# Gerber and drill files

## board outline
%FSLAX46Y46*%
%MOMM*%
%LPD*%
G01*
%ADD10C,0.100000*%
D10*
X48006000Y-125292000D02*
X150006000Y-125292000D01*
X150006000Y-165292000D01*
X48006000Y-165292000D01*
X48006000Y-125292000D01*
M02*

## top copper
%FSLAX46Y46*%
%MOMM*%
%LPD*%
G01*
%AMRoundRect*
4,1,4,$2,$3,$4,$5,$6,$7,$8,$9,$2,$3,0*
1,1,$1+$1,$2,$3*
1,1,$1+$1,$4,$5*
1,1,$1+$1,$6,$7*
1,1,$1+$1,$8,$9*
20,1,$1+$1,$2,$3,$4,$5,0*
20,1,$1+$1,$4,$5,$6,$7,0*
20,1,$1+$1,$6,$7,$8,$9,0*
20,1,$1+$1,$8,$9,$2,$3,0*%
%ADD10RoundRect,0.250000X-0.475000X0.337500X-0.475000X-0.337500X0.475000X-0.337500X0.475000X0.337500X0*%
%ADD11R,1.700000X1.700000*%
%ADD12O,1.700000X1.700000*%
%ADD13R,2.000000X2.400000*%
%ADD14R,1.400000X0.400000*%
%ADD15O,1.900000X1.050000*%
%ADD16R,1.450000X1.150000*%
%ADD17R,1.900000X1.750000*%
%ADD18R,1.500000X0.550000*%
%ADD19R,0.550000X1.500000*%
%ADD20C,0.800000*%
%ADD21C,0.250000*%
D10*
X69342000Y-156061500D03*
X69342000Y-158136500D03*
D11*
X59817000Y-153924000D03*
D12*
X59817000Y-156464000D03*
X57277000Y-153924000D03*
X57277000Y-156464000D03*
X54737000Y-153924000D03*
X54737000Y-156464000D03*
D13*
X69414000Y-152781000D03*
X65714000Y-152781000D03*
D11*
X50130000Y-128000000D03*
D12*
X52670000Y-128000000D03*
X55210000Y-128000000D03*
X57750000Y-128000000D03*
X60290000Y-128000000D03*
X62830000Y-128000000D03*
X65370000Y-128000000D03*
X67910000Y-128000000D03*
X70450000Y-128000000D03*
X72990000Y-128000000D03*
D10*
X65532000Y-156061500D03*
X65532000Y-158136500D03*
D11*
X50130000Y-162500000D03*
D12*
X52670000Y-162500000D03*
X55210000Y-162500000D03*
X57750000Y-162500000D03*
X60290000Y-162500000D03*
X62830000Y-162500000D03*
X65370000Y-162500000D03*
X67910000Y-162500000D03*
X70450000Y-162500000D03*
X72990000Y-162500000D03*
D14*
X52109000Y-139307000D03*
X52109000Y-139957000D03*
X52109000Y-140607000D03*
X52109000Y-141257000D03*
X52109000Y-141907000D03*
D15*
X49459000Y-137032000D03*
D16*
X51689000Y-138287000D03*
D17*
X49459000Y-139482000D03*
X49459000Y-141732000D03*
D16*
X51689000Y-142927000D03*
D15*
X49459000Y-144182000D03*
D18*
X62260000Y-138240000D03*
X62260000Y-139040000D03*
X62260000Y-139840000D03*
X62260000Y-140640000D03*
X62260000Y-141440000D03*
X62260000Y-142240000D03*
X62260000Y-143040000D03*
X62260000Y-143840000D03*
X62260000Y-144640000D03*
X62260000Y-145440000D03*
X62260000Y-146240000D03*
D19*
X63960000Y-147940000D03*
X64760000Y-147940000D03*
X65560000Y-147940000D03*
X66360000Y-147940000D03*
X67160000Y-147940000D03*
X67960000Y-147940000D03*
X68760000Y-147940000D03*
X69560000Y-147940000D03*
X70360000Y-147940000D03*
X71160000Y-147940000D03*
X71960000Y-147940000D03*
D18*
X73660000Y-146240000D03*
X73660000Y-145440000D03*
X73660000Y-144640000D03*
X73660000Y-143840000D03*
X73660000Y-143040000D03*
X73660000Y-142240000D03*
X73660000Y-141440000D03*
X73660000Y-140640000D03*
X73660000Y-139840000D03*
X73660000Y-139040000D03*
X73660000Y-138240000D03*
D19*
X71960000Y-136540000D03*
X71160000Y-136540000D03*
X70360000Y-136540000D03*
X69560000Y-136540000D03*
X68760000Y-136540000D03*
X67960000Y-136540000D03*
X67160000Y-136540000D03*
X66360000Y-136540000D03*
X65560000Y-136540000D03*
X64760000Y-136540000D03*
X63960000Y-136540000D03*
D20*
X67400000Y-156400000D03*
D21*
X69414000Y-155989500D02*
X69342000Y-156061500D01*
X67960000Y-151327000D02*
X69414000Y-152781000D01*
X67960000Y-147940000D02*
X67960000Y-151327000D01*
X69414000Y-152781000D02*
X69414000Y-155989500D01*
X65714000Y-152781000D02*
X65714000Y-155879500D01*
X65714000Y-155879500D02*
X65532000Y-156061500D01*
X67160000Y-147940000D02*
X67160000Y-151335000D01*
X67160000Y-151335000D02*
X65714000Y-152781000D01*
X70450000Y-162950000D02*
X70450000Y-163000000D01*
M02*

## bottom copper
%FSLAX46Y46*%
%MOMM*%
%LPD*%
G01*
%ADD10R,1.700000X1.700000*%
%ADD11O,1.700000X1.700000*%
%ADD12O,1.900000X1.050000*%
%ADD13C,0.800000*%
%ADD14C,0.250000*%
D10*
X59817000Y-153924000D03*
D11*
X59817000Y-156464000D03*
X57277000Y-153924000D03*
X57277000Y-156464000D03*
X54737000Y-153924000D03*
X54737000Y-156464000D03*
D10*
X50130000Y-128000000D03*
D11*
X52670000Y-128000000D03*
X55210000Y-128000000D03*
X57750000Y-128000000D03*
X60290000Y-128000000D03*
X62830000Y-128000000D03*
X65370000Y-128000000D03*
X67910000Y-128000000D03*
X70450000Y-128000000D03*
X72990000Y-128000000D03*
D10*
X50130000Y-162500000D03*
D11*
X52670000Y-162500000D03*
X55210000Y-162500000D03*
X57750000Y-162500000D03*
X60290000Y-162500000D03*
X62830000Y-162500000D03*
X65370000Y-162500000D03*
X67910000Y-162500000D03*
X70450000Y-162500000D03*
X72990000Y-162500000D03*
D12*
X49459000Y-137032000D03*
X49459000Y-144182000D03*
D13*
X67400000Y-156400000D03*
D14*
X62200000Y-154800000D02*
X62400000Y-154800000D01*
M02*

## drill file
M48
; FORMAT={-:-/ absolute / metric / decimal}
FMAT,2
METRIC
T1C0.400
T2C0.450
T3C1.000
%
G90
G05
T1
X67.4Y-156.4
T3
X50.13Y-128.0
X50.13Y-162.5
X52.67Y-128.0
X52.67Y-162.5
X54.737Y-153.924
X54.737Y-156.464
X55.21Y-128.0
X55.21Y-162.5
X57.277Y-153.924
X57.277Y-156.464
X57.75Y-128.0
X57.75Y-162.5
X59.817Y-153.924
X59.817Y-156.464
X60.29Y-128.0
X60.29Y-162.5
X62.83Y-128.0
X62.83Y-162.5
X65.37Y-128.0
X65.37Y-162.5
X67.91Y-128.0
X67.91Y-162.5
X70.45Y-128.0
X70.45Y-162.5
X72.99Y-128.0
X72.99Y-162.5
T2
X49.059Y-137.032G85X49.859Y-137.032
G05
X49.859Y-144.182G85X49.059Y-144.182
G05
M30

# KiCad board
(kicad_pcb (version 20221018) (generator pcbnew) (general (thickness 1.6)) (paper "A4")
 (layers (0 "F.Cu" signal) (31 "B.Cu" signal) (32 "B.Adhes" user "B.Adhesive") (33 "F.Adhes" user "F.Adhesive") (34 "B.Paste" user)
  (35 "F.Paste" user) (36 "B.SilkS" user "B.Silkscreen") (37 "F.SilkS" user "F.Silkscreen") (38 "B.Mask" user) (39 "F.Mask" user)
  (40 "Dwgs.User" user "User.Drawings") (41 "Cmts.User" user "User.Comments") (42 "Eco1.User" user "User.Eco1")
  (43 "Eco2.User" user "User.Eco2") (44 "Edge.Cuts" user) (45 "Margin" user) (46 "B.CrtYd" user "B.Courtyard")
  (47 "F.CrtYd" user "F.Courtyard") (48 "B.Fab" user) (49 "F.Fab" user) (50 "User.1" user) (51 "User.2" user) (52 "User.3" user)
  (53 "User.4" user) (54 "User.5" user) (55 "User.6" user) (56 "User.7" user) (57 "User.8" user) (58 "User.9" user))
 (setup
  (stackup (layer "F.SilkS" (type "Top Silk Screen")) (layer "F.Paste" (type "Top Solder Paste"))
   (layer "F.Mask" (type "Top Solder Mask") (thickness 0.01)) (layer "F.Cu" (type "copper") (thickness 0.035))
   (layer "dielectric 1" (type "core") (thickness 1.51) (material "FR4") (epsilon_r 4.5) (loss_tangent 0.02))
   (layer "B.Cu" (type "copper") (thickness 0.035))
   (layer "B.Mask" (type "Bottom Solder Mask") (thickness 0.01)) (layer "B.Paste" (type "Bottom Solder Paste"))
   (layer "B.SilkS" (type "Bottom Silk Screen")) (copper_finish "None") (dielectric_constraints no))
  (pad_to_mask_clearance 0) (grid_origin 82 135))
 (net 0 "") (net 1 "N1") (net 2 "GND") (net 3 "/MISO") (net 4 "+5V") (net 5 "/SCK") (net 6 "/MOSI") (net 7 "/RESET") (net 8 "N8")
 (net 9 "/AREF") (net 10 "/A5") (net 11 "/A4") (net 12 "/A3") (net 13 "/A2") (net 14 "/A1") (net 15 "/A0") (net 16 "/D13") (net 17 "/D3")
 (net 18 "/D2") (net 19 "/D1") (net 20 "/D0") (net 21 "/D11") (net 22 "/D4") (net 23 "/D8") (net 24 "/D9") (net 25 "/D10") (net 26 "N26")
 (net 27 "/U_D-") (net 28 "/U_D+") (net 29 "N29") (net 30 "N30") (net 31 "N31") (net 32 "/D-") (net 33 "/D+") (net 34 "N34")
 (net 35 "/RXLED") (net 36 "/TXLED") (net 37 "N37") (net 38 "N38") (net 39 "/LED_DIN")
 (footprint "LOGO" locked (layer "F.Cu") (at 125.95 162)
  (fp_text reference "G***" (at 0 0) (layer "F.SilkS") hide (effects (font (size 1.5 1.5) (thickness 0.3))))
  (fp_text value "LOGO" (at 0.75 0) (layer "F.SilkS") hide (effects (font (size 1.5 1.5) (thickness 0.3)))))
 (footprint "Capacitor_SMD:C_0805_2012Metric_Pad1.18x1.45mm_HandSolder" (layer "F.Cu") (at 69.342 157.099 -90)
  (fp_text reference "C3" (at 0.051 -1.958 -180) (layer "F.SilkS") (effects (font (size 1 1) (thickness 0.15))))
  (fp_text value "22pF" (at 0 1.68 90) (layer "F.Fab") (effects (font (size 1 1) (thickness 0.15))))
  (pad "1" smd roundrect (at -1.0375 0 270) (size 1.175 1.45) (layers "F.Cu" "F.Paste" "F.Mask") (roundrect_rratio 0.2127659574)
   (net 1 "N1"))
  (pad "2" smd roundrect (at 1.0375 0 270) (size 1.175 1.45) (layers "F.Cu" "F.Paste" "F.Mask") (roundrect_rratio 0.2127659574)
   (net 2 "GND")))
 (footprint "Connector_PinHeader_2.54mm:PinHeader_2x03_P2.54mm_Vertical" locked (layer "F.Cu") (at 59.817 153.924 -90)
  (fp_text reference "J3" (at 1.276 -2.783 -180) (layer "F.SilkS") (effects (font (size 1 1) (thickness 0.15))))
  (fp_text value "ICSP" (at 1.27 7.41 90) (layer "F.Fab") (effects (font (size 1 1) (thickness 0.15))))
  (pad "1" thru_hole rect locked (at 0 0 270) (size 1.7 1.7) (drill 1) (layers "*.Cu" "*.Mask") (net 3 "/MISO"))
  (pad "2" thru_hole oval locked (at 2.54 0 270) (size 1.7 1.7) (drill 1) (layers "*.Cu" "*.Mask") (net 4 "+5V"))
  (pad "3" thru_hole oval locked (at 0 2.54 270) (size 1.7 1.7) (drill 1) (layers "*.Cu" "*.Mask") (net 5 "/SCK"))
  (pad "4" thru_hole oval locked (at 2.54 2.54 270) (size 1.7 1.7) (drill 1) (layers "*.Cu" "*.Mask") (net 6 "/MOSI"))
  (pad "5" thru_hole oval locked (at 0 5.08 270) (size 1.7 1.7) (drill 1) (layers "*.Cu" "*.Mask") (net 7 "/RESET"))
  (pad "6" thru_hole oval locked (at 2.54 5.08 270) (size 1.7 1.7) (drill 1) (layers "*.Cu" "*.Mask") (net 2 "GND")))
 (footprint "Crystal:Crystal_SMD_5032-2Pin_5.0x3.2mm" (layer "F.Cu") (at 67.564 152.781 180)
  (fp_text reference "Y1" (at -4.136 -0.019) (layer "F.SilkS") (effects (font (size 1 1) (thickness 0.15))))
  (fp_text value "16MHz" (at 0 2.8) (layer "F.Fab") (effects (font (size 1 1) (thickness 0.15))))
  (pad "1" smd rect (at -1.85 0 180) (size 2 2.4) (layers "F.Cu" "F.Paste" "F.Mask") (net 1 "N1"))
  (pad "2" smd rect (at 1.85 0 180) (size 2 2.4) (layers "F.Cu" "F.Paste" "F.Mask") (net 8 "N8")))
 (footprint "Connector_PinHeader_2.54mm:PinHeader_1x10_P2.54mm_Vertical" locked (layer "F.Cu") (at 50.13 128 90)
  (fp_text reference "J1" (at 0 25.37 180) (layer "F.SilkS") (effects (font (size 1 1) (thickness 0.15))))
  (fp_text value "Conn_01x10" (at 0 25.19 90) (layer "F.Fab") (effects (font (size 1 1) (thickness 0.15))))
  (pad "1" thru_hole rect locked (at 0 0 90) (size 1.7 1.7) (drill 1) (layers "*.Cu" "*.Mask") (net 4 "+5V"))
  (pad "2" thru_hole oval locked (at 0 2.54 90) (size 1.7 1.7) (drill 1) (layers "*.Cu" "*.Mask") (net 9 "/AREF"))
  (pad "3" thru_hole oval locked (at 0 5.08 90) (size 1.7 1.7) (drill 1) (layers "*.Cu" "*.Mask") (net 2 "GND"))
  (pad "4" thru_hole oval locked (at 0 7.62 90) (size 1.7 1.7) (drill 1) (layers "*.Cu" "*.Mask") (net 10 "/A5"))
  (pad "5" thru_hole oval locked (at 0 10.16 90) (size 1.7 1.7) (drill 1) (layers "*.Cu" "*.Mask") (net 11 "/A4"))
  (pad "6" thru_hole oval locked (at 0 12.7 90) (size 1.7 1.7) (drill 1) (layers "*.Cu" "*.Mask") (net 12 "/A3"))
  (pad "7" thru_hole oval locked (at 0 15.24 90) (size 1.7 1.7) (drill 1) (layers "*.Cu" "*.Mask") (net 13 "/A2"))
  (pad "8" thru_hole oval locked (at 0 17.78 90) (size 1.7 1.7) (drill 1) (layers "*.Cu" "*.Mask") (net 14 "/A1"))
  (pad "9" thru_hole oval locked (at 0 20.32 90) (size 1.7 1.7) (drill 1) (layers "*.Cu" "*.Mask") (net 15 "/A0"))
  (pad "10" thru_hole oval locked (at 0 22.86 90) (size 1.7 1.7) (drill 1) (layers "*.Cu" "*.Mask") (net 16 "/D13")))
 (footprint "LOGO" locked (layer "F.Cu") (at 142.15 161.8)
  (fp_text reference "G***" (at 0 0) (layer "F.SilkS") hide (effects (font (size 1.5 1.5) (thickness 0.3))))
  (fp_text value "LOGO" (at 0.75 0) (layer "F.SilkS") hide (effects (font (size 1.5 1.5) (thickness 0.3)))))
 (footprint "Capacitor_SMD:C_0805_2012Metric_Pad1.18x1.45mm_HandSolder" (layer "F.Cu") (at 65.532 157.099 -90)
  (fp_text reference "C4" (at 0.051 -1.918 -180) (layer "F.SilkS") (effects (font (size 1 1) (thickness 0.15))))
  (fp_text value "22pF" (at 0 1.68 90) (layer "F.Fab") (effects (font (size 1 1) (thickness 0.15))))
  (pad "1" smd roundrect (at -1.0375 0 270) (size 1.175 1.45) (layers "F.Cu" "F.Paste" "F.Mask") (roundrect_rratio 0.2127659574)
   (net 8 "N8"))
  (pad "2" smd roundrect (at 1.0375 0 270) (size 1.175 1.45) (layers "F.Cu" "F.Paste" "F.Mask") (roundrect_rratio 0.2127659574)
   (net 2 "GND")))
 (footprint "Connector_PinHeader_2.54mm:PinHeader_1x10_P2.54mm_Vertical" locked (layer "F.Cu") (at 50.13 162.5 90)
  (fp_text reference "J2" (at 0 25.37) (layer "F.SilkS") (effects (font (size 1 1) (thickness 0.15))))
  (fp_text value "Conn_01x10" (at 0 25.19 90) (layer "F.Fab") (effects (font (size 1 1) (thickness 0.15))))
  (pad "1" thru_hole rect locked (at 0 0 90) (size 1.7 1.7) (drill 1) (layers "*.Cu" "*.Mask") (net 2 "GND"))
  (pad "2" thru_hole oval locked (at 0 2.54 90) (size 1.7 1.7) (drill 1) (layers "*.Cu" "*.Mask") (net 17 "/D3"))
  (pad "3" thru_hole oval locked (at 0 5.08 90) (size 1.7 1.7) (drill 1) (layers "*.Cu" "*.Mask") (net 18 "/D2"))
  (pad "4" thru_hole oval locked (at 0 7.62 90) (size 1.7 1.7) (drill 1) (layers "*.Cu" "*.Mask") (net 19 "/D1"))
  (pad "5" thru_hole oval locked (at 0 10.16 90) (size 1.7 1.7) (drill 1) (layers "*.Cu" "*.Mask") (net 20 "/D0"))
  (pad "6" thru_hole oval locked (at 0 12.7 90) (size 1.7 1.7) (drill 1) (layers "*.Cu" "*.Mask") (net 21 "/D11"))
  (pad "7" thru_hole oval locked (at 0 15.24 90) (size 1.7 1.7) (drill 1) (layers "*.Cu" "*.Mask") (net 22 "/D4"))
  (pad "8" thru_hole oval locked (at 0 17.78 90) (size 1.7 1.7) (drill 1) (layers "*.Cu" "*.Mask") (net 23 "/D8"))
  (pad "9" thru_hole oval locked (at 0 20.32 90) (size 1.7 1.7) (drill 1) (layers "*.Cu" "*.Mask") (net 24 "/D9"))
  (pad "10" thru_hole oval locked (at 0 22.86 90) (size 1.7 1.7) (drill 1) (layers "*.Cu" "*.Mask") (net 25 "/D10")))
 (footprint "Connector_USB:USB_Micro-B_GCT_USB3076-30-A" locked (layer "F.Cu") (at 50.659 140.607 -90)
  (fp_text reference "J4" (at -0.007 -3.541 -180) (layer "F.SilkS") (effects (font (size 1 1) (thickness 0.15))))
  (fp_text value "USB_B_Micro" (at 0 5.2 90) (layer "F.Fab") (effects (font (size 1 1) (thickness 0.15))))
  (pad "1" smd rect locked (at -1.3 -1.45 270) (size 0.4 1.4) (layers "F.Cu" "F.Paste" "F.Mask") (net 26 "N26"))
  (pad "2" smd rect locked (at -0.65 -1.45 270) (size 0.4 1.4) (layers "F.Cu" "F.Paste" "F.Mask") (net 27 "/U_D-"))
  (pad "3" smd rect locked (at 0 -1.45 270) (size 0.4 1.4) (layers "F.Cu" "F.Paste" "F.Mask") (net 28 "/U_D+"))
  (pad "4" smd rect locked (at 0.65 -1.45 270) (size 0.4 1.4) (layers "F.Cu" "F.Paste" "F.Mask") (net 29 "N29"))
  (pad "5" smd rect locked (at 1.3 -1.45 270) (size 0.4 1.4) (layers "F.Cu" "F.Paste" "F.Mask") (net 2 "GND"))
  (pad "6" thru_hole oval locked (at -3.575 1.2 90) (size 1.05 1.9) (drill oval 0.45 1.25) (layers "*.Cu" "*.Mask") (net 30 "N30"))
  (pad "6" smd rect locked (at -2.32 -1.03 270) (size 1.15 1.45) (layers "F.Cu" "F.Paste" "F.Mask") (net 30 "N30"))
  (pad "6" smd rect locked (at -1.125 1.2 270) (size 1.75 1.9) (layers "F.Cu" "F.Paste" "F.Mask") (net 30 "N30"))
  (pad "6" smd rect locked (at 1.125 1.2 270) (size 1.75 1.9) (layers "F.Cu" "F.Paste" "F.Mask") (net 30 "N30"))
  (pad "6" smd rect locked (at 2.32 -1.03 270) (size 1.15 1.45) (layers "F.Cu" "F.Paste" "F.Mask") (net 30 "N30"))
  (pad "6" thru_hole oval locked (at 3.575 1.2 270) (size 1.05 1.9) (drill oval 0.45 1.25) (layers "*.Cu" "*.Mask") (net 30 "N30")))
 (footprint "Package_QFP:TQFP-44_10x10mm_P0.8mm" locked (layer "F.Cu") (at 67.96 142.24)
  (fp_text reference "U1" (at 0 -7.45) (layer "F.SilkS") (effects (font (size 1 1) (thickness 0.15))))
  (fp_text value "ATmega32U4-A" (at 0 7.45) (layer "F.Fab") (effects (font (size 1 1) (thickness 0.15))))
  (pad "1" smd rect locked (at -5.7 -4) (size 1.5 0.55) (layers "F.Cu" "F.Paste" "F.Mask") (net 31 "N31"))
  (pad "2" smd rect locked (at -5.7 -3.2) (size 1.5 0.55) (layers "F.Cu" "F.Paste" "F.Mask") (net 4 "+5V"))
  (pad "3" smd rect locked (at -5.7 -2.4) (size 1.5 0.55) (layers "F.Cu" "F.Paste" "F.Mask") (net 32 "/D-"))
  (pad "4" smd rect locked (at -5.7 -1.6) (size 1.5 0.55) (layers "F.Cu" "F.Paste" "F.Mask") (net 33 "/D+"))
  (pad "5" smd rect locked (at -5.7 -0.8) (size 1.5 0.55) (layers "F.Cu" "F.Paste" "F.Mask") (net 2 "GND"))
  (pad "6" smd rect locked (at -5.7 0) (size 1.5 0.55) (layers "F.Cu" "F.Paste" "F.Mask") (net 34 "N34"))
  (pad "7" smd rect locked (at -5.7 0.8) (size 1.5 0.55) (layers "F.Cu" "F.Paste" "F.Mask") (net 4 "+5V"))
  (pad "8" smd rect locked (at -5.7 1.6) (size 1.5 0.55) (layers "F.Cu" "F.Paste" "F.Mask") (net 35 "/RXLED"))
  (pad "9" smd rect locked (at -5.7 2.4) (size 1.5 0.55) (layers "F.Cu" "F.Paste" "F.Mask") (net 5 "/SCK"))
  (pad "10" smd rect locked (at -5.7 3.2) (size 1.5 0.55) (layers "F.Cu" "F.Paste" "F.Mask") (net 6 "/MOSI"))
  (pad "11" smd rect locked (at -5.7 4) (size 1.5 0.55) (layers "F.Cu" "F.Paste" "F.Mask") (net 3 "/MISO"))
  (pad "12" smd rect locked (at -4 5.7 90) (size 1.5 0.55) (layers "F.Cu" "F.Paste" "F.Mask") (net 21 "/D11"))
  (pad "13" smd rect locked (at -3.2 5.7 90) (size 1.5 0.55) (layers "F.Cu" "F.Paste" "F.Mask") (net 7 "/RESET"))
  (pad "14" smd rect locked (at -2.4 5.7 90) (size 1.5 0.55) (layers "F.Cu" "F.Paste" "F.Mask") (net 4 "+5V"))
  (pad "15" smd rect locked (at -1.6 5.7 90) (size 1.5 0.55) (layers "F.Cu" "F.Paste" "F.Mask") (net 2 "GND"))
  (pad "16" smd rect locked (at -0.8 5.7 90) (size 1.5 0.55) (layers "F.Cu" "F.Paste" "F.Mask") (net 8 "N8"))
  (pad "17" smd rect locked (at 0 5.7 90) (size 1.5 0.55) (layers "F.Cu" "F.Paste" "F.Mask") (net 1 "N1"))
  (pad "18" smd rect locked (at 0.8 5.7 90) (size 1.5 0.55) (layers "F.Cu" "F.Paste" "F.Mask") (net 17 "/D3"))
  (pad "19" smd rect locked (at 1.6 5.7 90) (size 1.5 0.55) (layers "F.Cu" "F.Paste" "F.Mask") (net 18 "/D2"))
  (pad "20" smd rect locked (at 2.4 5.7 90) (size 1.5 0.55) (layers "F.Cu" "F.Paste" "F.Mask") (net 20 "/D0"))
  (pad "21" smd rect locked (at 3.2 5.7 90) (size 1.5 0.55) (layers "F.Cu" "F.Paste" "F.Mask") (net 19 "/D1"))
  (pad "22" smd rect locked (at 4 5.7 90) (size 1.5 0.55) (layers "F.Cu" "F.Paste" "F.Mask") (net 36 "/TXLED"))
  (pad "23" smd rect locked (at 5.7 4) (size 1.5 0.55) (layers "F.Cu" "F.Paste" "F.Mask") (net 2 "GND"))
  (pad "24" smd rect locked (at 5.7 3.2) (size 1.5 0.55) (layers "F.Cu" "F.Paste" "F.Mask") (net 4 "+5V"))
  (pad "25" smd rect locked (at 5.7 2.4) (size 1.5 0.55) (layers "F.Cu" "F.Paste" "F.Mask") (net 22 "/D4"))
  (pad "26" smd rect locked (at 5.7 1.6) (size 1.5 0.55) (layers "F.Cu" "F.Paste" "F.Mask") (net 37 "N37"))
  (pad "27" smd rect locked (at 5.7 0.8) (size 1.5 0.55) (layers "F.Cu" "F.Paste" "F.Mask") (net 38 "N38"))
  (pad "28" smd rect locked (at 5.7 0) (size 1.5 0.55) (layers "F.Cu" "F.Paste" "F.Mask") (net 23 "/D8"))
  (pad "29" smd rect locked (at 5.7 -0.8) (size 1.5 0.55) (layers "F.Cu" "F.Paste" "F.Mask") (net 24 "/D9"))
  (pad "30" smd rect locked (at 5.7 -1.6) (size 1.5 0.55) (layers "F.Cu" "F.Paste" "F.Mask") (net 25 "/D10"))
  (pad "31" smd rect locked (at 5.7 -2.4) (size 1.5 0.55) (layers "F.Cu" "F.Paste" "F.Mask") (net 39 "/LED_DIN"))
  (pad "32" smd rect locked (at 5.7 -3.2) (size 1.5 0.55) (layers "F.Cu" "F.Paste" "F.Mask") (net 16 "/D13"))
  (pad "33" smd rect locked (at 5.7 -4) (size 1.5 0.55) (layers "F.Cu" "F.Paste" "F.Mask") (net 2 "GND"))
  (pad "34" smd rect locked (at 4 -5.7 90) (size 1.5 0.55) (layers "F.Cu" "F.Paste" "F.Mask") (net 4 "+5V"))
  (pad "35" smd rect locked (at 3.2 -5.7 90) (size 1.5 0.55) (layers "F.Cu" "F.Paste" "F.Mask") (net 2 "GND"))
  (pad "36" smd rect locked (at 2.4 -5.7 90) (size 1.5 0.55) (layers "F.Cu" "F.Paste" "F.Mask") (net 15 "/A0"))
  (pad "37" smd rect locked (at 1.6 -5.7 90) (size 1.5 0.55) (layers "F.Cu" "F.Paste" "F.Mask") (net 14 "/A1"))
  (pad "38" smd rect locked (at 0.8 -5.7 90) (size 1.5 0.55) (layers "F.Cu" "F.Paste" "F.Mask") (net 13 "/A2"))
  (pad "39" smd rect locked (at 0 -5.7 90) (size 1.5 0.55) (layers "F.Cu" "F.Paste" "F.Mask") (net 12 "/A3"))
  (pad "40" smd rect locked (at -0.8 -5.7 90) (size 1.5 0.55) (layers "F.Cu" "F.Paste" "F.Mask") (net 11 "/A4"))
  (pad "41" smd rect locked (at -1.6 -5.7 90) (size 1.5 0.55) (layers "F.Cu" "F.Paste" "F.Mask") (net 10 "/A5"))
  (pad "42" smd rect locked (at -2.4 -5.7 90) (size 1.5 0.55) (layers "F.Cu" "F.Paste" "F.Mask") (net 9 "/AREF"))
  (pad "43" smd rect locked (at -3.2 -5.7 90) (size 1.5 0.55) (layers "F.Cu" "F.Paste" "F.Mask") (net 2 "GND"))
  (pad "44" smd rect locked (at -4 -5.7 90) (size 1.5 0.55) (layers "F.Cu" "F.Paste" "F.Mask") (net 4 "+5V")))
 (gr_rect (start 48.006 125.292) (end 150.006 165.292) (stroke (width 0.1) (type default)) (fill none) (layer "Edge.Cuts"))
 (via (at 67.4 156.4) (size 0.8) (drill 0.4) (layers "F.Cu" "B.Cu") (free) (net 2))
 (segment (start 69.414 155.9895) (end 69.342 156.0615) (width 0.25) (layer "F.Cu") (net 1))
 (segment (start 67.96 151.327) (end 69.414 152.781) (width 0.25) (layer "F.Cu") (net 1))
 (segment (start 67.96 147.94) (end 67.96 151.327) (width 0.25) (layer "F.Cu") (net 1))
 (segment (start 69.414 152.781) (end 69.414 155.9895) (width 0.25) (layer "F.Cu") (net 1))
 (segment (start 65.714 152.781) (end 65.714 155.8795) (width 0.25) (layer "F.Cu") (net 8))
 (segment (start 65.714 155.8795) (end 65.532 156.0615) (width 0.25) (layer "F.Cu") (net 8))
 (segment (start 67.16 147.94) (end 67.16 151.335) (width 0.25) (layer "F.Cu") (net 8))
 (segment (start 67.16 151.335) (end 65.714 152.781) (width 0.25) (layer "F.Cu") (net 8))
 (segment (start 62.2 154.8) (end 62.4 154.8) (width 0.25) (layer "B.Cu") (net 21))
 (segment (start 70.45 162.95) (end 70.45 163) (width 0.25) (layer "F.Cu") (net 24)))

